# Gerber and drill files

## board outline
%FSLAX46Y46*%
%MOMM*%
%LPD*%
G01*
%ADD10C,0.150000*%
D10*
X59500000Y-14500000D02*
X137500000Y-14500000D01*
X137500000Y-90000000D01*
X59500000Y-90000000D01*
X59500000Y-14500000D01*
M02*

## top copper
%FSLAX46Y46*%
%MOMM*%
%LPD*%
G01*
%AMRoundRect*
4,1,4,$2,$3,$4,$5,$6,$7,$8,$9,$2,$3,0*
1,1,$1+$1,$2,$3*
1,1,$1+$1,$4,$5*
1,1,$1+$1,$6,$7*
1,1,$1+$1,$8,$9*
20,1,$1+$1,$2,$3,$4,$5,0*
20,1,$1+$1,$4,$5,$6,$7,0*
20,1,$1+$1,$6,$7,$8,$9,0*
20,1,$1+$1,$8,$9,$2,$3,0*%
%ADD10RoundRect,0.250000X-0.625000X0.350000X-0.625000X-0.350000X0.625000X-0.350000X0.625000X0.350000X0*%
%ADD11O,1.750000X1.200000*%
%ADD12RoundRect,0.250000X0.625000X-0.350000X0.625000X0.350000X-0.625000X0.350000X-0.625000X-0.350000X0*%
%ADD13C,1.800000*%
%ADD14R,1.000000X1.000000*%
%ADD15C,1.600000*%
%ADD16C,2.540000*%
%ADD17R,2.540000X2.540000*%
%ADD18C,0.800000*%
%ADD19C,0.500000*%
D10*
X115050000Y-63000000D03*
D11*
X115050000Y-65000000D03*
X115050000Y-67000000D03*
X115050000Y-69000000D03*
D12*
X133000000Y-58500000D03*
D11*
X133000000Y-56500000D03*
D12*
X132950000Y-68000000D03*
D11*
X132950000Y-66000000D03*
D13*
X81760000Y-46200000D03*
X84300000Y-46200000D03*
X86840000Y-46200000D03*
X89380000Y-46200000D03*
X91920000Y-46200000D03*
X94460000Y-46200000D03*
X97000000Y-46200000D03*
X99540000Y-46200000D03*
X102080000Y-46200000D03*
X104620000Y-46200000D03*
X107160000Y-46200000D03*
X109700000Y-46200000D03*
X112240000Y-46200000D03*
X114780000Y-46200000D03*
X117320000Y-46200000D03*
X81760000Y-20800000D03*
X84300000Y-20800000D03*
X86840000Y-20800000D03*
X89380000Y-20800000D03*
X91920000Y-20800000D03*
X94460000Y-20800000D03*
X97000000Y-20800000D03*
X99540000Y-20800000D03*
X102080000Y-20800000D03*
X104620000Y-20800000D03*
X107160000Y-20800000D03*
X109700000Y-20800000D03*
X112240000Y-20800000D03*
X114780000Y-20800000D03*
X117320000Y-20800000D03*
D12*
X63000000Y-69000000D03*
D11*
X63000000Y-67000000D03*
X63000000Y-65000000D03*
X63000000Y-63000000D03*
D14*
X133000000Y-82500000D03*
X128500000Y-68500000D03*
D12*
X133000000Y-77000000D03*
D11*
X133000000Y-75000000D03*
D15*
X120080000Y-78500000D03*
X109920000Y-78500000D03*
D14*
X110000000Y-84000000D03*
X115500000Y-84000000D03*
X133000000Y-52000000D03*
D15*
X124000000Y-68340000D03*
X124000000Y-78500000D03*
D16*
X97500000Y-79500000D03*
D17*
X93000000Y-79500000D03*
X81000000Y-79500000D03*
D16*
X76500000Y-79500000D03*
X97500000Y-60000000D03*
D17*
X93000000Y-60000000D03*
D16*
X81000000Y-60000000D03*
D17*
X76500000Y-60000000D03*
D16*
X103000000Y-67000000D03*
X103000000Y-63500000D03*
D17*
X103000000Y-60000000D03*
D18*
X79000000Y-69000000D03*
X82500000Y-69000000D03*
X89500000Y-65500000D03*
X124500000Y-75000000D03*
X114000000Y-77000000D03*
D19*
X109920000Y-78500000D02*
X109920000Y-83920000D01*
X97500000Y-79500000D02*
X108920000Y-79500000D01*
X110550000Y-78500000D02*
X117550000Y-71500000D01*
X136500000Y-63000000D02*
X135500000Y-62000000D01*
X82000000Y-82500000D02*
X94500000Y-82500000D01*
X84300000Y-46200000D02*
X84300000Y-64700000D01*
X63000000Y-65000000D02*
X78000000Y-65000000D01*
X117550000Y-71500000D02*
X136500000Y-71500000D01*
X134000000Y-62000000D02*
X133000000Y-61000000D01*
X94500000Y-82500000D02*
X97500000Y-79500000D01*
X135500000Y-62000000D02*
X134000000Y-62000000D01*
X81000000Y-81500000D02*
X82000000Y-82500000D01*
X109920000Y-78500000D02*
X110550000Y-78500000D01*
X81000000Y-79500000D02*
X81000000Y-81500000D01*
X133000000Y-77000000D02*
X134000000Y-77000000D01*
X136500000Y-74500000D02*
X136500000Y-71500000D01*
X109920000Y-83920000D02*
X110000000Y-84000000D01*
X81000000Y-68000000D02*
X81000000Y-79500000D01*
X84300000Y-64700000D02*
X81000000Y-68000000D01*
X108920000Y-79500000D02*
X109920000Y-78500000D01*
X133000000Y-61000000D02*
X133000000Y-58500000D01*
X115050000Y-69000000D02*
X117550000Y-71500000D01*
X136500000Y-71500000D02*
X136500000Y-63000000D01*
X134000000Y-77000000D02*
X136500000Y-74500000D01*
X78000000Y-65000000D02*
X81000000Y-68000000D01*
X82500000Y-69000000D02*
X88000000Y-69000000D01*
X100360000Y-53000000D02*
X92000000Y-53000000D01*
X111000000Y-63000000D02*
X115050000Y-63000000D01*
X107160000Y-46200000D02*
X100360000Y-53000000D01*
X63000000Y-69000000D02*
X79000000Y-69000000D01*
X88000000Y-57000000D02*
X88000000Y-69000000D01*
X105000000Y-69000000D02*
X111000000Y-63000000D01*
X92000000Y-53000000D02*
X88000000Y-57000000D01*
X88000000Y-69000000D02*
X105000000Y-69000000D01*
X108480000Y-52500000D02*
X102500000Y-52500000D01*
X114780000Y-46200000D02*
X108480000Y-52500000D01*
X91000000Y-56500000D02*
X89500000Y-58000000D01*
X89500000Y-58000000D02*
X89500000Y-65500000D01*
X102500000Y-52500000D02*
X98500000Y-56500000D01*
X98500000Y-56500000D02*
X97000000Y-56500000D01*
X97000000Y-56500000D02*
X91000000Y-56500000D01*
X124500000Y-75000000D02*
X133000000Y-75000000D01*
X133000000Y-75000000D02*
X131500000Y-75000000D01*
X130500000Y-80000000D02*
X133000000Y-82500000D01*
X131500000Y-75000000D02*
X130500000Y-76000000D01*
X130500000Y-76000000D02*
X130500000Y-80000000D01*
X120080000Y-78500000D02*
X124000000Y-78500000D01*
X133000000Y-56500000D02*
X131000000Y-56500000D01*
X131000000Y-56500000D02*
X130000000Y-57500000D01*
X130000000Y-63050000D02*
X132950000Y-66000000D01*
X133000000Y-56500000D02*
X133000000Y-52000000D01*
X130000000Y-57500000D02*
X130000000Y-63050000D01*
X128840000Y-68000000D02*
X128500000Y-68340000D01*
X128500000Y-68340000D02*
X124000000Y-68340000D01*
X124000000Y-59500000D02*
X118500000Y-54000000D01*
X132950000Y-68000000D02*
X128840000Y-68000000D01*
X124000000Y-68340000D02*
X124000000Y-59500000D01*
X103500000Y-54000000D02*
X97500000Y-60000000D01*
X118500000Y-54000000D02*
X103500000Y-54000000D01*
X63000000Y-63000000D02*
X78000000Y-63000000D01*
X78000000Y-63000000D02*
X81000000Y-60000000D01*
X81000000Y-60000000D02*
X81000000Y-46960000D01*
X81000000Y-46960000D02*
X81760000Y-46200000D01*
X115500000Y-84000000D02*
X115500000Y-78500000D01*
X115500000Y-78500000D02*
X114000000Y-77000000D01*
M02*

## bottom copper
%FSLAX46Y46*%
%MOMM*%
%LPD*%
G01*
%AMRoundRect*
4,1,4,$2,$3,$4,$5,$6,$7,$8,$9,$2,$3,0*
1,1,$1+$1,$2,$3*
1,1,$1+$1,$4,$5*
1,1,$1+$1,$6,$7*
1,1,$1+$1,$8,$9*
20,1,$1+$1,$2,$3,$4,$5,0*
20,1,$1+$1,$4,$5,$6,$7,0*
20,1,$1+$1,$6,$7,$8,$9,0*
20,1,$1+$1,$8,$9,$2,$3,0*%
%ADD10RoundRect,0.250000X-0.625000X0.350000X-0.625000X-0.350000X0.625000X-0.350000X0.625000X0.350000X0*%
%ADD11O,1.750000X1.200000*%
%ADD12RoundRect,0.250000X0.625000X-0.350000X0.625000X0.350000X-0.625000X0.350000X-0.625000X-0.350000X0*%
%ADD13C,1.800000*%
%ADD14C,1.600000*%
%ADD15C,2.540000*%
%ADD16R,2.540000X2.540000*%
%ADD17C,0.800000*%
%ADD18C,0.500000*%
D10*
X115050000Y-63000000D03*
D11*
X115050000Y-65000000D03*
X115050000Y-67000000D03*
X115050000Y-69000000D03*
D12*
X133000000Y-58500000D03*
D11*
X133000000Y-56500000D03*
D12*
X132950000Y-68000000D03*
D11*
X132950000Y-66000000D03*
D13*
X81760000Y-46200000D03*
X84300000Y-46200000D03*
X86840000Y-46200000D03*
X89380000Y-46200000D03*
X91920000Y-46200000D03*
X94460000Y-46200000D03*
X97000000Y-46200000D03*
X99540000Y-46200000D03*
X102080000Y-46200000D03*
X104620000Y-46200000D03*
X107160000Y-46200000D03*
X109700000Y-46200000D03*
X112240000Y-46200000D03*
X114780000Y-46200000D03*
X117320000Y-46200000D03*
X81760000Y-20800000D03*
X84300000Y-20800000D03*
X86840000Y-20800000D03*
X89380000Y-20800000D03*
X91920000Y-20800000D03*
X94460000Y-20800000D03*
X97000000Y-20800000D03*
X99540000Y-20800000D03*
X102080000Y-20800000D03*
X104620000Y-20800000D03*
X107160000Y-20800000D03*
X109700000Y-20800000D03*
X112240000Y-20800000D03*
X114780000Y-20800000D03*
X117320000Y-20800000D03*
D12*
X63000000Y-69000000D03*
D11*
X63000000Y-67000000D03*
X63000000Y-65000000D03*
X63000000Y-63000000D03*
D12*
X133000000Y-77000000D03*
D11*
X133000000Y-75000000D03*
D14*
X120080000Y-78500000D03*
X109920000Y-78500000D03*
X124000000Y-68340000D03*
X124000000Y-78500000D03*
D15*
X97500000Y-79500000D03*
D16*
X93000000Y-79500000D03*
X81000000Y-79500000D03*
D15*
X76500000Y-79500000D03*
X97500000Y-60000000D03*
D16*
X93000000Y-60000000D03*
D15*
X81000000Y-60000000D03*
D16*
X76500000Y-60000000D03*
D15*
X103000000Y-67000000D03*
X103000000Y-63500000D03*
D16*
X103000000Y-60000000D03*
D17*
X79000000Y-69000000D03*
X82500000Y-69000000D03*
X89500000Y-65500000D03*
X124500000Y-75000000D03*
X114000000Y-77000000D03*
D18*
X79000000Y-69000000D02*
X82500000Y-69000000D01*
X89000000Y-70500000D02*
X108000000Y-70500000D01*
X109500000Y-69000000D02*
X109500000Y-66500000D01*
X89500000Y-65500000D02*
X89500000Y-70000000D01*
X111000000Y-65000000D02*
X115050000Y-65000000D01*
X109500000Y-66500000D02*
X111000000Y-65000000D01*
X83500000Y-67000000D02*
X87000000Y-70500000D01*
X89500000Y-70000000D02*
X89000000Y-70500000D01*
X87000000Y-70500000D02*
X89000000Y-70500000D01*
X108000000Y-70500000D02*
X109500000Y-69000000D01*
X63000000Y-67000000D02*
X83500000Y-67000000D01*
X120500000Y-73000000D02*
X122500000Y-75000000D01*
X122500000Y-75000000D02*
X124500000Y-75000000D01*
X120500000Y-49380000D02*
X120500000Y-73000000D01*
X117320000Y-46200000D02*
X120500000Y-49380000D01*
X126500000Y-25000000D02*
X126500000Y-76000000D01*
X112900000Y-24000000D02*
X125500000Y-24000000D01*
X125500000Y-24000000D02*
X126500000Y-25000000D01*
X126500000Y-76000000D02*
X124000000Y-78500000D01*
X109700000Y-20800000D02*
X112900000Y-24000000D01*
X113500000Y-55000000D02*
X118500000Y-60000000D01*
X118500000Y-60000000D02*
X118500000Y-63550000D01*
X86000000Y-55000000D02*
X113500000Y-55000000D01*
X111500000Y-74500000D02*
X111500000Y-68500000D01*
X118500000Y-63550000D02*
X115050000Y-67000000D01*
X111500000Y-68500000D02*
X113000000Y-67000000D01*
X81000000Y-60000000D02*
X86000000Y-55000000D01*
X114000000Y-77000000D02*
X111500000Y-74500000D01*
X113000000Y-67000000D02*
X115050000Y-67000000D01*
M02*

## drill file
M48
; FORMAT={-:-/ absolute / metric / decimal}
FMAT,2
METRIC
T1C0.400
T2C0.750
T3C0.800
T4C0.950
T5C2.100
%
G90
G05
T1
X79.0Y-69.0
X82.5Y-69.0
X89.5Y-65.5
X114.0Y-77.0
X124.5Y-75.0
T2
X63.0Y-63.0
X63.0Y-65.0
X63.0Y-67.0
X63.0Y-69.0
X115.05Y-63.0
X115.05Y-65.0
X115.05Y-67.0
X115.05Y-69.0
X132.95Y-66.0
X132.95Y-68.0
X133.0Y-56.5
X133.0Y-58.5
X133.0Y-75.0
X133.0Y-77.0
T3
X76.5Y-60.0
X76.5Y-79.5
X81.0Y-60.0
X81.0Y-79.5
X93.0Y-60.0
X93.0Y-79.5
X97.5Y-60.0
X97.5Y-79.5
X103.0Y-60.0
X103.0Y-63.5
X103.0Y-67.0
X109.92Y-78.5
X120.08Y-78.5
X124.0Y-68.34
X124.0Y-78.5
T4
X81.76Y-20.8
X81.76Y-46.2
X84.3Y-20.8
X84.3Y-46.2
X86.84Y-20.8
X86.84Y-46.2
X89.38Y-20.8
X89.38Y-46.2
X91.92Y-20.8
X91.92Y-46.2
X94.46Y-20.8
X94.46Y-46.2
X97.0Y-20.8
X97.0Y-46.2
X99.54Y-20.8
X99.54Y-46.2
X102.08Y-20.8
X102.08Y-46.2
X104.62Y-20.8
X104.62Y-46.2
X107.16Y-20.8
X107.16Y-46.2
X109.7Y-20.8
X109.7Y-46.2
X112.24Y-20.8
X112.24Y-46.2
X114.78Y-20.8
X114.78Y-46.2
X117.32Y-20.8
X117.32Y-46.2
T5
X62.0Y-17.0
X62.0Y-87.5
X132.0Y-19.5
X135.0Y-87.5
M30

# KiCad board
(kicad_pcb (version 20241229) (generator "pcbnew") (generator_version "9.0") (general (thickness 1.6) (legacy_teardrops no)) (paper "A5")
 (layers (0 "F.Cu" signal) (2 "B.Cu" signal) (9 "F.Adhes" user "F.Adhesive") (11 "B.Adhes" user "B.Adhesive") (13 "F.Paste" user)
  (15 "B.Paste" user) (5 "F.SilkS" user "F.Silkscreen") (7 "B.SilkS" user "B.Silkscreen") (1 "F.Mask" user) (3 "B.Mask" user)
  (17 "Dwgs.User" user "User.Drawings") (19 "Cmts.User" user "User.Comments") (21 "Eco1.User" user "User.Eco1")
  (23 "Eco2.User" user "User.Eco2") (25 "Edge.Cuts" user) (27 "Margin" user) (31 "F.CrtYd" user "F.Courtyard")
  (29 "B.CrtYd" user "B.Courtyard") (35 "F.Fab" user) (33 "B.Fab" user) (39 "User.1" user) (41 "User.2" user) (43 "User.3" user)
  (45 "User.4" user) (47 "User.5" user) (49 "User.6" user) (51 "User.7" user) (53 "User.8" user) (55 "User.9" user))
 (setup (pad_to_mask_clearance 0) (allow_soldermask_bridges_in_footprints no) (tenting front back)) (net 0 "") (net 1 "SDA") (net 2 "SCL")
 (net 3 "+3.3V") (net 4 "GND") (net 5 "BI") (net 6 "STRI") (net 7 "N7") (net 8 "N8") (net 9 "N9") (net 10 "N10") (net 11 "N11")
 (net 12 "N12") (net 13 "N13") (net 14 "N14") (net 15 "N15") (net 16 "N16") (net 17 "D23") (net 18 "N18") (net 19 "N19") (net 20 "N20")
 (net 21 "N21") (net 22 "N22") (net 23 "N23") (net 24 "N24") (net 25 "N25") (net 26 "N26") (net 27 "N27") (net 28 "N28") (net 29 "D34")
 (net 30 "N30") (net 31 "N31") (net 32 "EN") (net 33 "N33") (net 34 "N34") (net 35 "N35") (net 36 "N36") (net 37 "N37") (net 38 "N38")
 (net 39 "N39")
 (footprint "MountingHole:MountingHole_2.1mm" (layer "F.Cu") (at 62 17)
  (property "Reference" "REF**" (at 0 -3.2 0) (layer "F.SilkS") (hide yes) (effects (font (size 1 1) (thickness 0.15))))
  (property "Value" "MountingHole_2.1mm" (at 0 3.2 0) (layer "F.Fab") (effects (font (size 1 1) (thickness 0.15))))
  (pad "" np_thru_hole circle (at 0 0) (size 2.1 2.1) (drill 2.1) (layers "*.Cu" "*.Mask")))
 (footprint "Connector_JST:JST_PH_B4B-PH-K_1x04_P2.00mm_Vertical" (layer "F.Cu") (at 115.05 63 -90)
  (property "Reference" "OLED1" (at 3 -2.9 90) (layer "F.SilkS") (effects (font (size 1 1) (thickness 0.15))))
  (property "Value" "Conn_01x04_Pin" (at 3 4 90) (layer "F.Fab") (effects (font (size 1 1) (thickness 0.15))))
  (pad "1" thru_hole roundrect (at 0 0 270) (size 1.2 1.75) (drill 0.75) (layers "*.Cu" "*.Mask") (remove_unused_layers no)
   (roundrect_rratio 0.208333) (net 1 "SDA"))
  (pad "2" thru_hole oval (at 2 0 270) (size 1.2 1.75) (drill 0.75) (layers "*.Cu" "*.Mask") (remove_unused_layers no) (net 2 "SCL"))
  (pad "3" thru_hole oval (at 4 0 270) (size 1.2 1.75) (drill 0.75) (layers "*.Cu" "*.Mask") (remove_unused_layers no) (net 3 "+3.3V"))
  (pad "4" thru_hole oval (at 6 0 270) (size 1.2 1.75) (drill 0.75) (layers "*.Cu" "*.Mask") (remove_unused_layers no) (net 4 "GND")))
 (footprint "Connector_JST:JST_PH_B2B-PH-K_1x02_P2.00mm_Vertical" (layer "F.Cu") (at 133 58.5 90)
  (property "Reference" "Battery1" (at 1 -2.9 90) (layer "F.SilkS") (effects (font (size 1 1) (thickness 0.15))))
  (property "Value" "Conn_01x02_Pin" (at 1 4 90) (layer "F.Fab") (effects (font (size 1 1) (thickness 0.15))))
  (pad "1" thru_hole roundrect (at 0 0 90) (size 1.2 1.75) (drill 0.75) (layers "*.Cu" "*.Mask") (remove_unused_layers no)
   (roundrect_rratio 0.208333) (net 4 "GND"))
  (pad "2" thru_hole oval (at 2 0 90) (size 1.2 1.75) (drill 0.75) (layers "*.Cu" "*.Mask") (remove_unused_layers no) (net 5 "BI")))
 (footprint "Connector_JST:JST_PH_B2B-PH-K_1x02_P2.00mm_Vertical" (layer "F.Cu") (at 132.95 68 90)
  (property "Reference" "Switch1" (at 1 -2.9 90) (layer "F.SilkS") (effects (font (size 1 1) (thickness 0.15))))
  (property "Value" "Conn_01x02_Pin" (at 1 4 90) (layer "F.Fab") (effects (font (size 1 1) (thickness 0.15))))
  (pad "1" thru_hole roundrect (at 0 0 90) (size 1.2 1.75) (drill 0.75) (layers "*.Cu" "*.Mask") (remove_unused_layers no)
   (roundrect_rratio 0.208333) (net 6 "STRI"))
  (pad "2" thru_hole oval (at 2 0 90) (size 1.2 1.75) (drill 0.75) (layers "*.Cu" "*.Mask") (remove_unused_layers no) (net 5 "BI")))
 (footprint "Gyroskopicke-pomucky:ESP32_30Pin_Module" (layer "F.Cu") (at 104.62 28.42 90)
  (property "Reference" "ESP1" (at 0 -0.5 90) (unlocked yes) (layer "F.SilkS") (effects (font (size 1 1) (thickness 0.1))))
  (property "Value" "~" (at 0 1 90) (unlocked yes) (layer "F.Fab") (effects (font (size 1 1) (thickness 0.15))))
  (pad "1" thru_hole circle (at -17.78 -22.86 90) (size 1.8 1.8) (drill 0.95) (layers "*.Cu" "*.Mask") (remove_unused_layers no)
   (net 3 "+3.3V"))
  (pad "2" thru_hole circle (at -17.78 -20.32 90) (size 1.8 1.8) (drill 0.95) (layers "*.Cu" "*.Mask") (remove_unused_layers no)
   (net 4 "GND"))
  (pad "3" thru_hole circle (at -17.78 -17.78 90) (size 1.8 1.8) (drill 0.95) (layers "*.Cu" "*.Mask") (remove_unused_layers no)
   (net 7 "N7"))
  (pad "4" thru_hole circle (at -17.78 -15.24 90) (size 1.8 1.8) (drill 0.95) (layers "*.Cu" "*.Mask") (remove_unused_layers no)
   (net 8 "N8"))
  (pad "5" thru_hole circle (at -17.78 -12.7 90) (size 1.8 1.8) (drill 0.95) (layers "*.Cu" "*.Mask") (remove_unused_layers no) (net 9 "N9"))
  (pad "6" thru_hole circle (at -17.78 -10.16 90) (size 1.8 1.8) (drill 0.95) (layers "*.Cu" "*.Mask") (remove_unused_layers no)
   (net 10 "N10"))
  (pad "7" thru_hole circle (at -17.78 -7.62 90) (size 1.8 1.8) (drill 0.95) (layers "*.Cu" "*.Mask") (remove_unused_layers no)
   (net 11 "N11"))
  (pad "8" thru_hole circle (at -17.78 -5.08 90) (size 1.8 1.8) (drill 0.95) (layers "*.Cu" "*.Mask") (remove_unused_layers no)
   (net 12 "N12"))
  (pad "9" thru_hole circle (at -17.78 -2.54 90) (size 1.8 1.8) (drill 0.95) (layers "*.Cu" "*.Mask") (remove_unused_layers no)
   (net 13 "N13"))
  (pad "10" thru_hole circle (at -17.78 0 90) (size 1.8 1.8) (drill 0.95) (layers "*.Cu" "*.Mask") (remove_unused_layers no) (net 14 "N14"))
  (pad "11" thru_hole circle (at -17.78 2.54 90) (size 1.8 1.8) (drill 0.95) (layers "*.Cu" "*.Mask") (remove_unused_layers no)
   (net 1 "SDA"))
  (pad "12" thru_hole circle (at -17.78 5.08 90) (size 1.8 1.8) (drill 0.95) (layers "*.Cu" "*.Mask") (remove_unused_layers no)
   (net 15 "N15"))
  (pad "13" thru_hole circle (at -17.78 7.62 90) (size 1.8 1.8) (drill 0.95) (layers "*.Cu" "*.Mask") (remove_unused_layers no)
   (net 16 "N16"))
  (pad "14" thru_hole circle (at -17.78 10.16 90) (size 1.8 1.8) (drill 0.95) (layers "*.Cu" "*.Mask") (remove_unused_layers no)
   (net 2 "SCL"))
  (pad "15" thru_hole circle (at -17.78 12.7 90) (size 1.8 1.8) (drill 0.95) (layers "*.Cu" "*.Mask") (remove_unused_layers no)
   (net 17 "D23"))
  (pad "16" thru_hole circle (at 7.62 -22.86 90) (size 1.8 1.8) (drill 0.95) (layers "*.Cu" "*.Mask") (remove_unused_layers no)
   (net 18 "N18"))
  (pad "17" thru_hole circle (at 7.62 -20.32 90) (size 1.8 1.8) (drill 0.95) (layers "*.Cu" "*.Mask") (remove_unused_layers no)
   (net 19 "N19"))
  (pad "18" thru_hole circle (at 7.62 -17.78 90) (size 1.8 1.8) (drill 0.95) (layers "*.Cu" "*.Mask") (remove_unused_layers no)
   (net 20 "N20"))
  (pad "19" thru_hole circle (at 7.62 -15.24 90) (size 1.8 1.8) (drill 0.95) (layers "*.Cu" "*.Mask") (remove_unused_layers no)
   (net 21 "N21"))
  (pad "20" thru_hole circle (at 7.62 -12.7 90) (size 1.8 1.8) (drill 0.95) (layers "*.Cu" "*.Mask") (remove_unused_layers no)
   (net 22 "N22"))
  (pad "21" thru_hole circle (at 7.62 -10.16 90) (size 1.8 1.8) (drill 0.95) (layers "*.Cu" "*.Mask") (remove_unused_layers no)
   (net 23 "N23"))
  (pad "22" thru_hole circle (at 7.62 -7.62 90) (size 1.8 1.8) (drill 0.95) (layers "*.Cu" "*.Mask") (remove_unused_layers no)
   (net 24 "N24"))
  (pad "23" thru_hole circle (at 7.62 -5.08 90) (size 1.8 1.8) (drill 0.95) (layers "*.Cu" "*.Mask") (remove_unused_layers no)
   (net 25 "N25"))
  (pad "24" thru_hole circle (at 7.62 -2.54 90) (size 1.8 1.8) (drill 0.95) (layers "*.Cu" "*.Mask") (remove_unused_layers no)
   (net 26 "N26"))
  (pad "25" thru_hole circle (at 7.62 0 90) (size 1.8 1.8) (drill 0.95) (layers "*.Cu" "*.Mask") (remove_unused_layers no) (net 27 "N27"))
  (pad "26" thru_hole circle (at 7.62 2.54 90) (size 1.8 1.8) (drill 0.95) (layers "*.Cu" "*.Mask") (remove_unused_layers no) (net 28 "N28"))
  (pad "27" thru_hole circle (at 7.62 5.08 90) (size 1.8 1.8) (drill 0.95) (layers "*.Cu" "*.Mask") (remove_unused_layers no) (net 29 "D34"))
  (pad "28" thru_hole circle (at 7.62 7.62 90) (size 1.8 1.8) (drill 0.95) (layers "*.Cu" "*.Mask") (remove_unused_layers no) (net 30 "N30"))
  (pad "29" thru_hole circle (at 7.62 10.16 90) (size 1.8 1.8) (drill 0.95) (layers "*.Cu" "*.Mask") (remove_unused_layers no)
   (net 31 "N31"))
  (pad "30" thru_hole circle (at 7.62 12.7 90) (size 1.8 1.8) (drill 0.95) (layers "*.Cu" "*.Mask") (remove_unused_layers no) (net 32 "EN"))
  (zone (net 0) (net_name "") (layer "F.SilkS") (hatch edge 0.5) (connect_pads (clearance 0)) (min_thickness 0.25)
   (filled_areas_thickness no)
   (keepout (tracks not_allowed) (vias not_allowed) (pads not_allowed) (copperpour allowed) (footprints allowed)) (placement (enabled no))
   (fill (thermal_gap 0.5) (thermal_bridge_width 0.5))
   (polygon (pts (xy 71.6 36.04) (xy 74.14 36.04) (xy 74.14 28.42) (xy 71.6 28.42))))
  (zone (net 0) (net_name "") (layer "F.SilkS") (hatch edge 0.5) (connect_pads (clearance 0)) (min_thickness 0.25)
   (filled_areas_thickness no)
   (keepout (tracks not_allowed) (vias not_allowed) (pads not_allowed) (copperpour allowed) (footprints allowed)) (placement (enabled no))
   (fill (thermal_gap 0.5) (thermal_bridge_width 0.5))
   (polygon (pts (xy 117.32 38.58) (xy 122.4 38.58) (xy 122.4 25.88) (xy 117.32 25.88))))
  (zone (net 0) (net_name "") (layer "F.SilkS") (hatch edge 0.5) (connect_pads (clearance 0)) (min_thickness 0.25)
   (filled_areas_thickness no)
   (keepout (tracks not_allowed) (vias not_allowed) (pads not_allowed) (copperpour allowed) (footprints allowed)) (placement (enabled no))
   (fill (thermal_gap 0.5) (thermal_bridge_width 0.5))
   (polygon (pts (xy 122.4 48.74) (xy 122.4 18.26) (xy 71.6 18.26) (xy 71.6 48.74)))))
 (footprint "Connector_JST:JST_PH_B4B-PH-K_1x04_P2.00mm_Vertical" (layer "F.Cu") (at 63 69 90)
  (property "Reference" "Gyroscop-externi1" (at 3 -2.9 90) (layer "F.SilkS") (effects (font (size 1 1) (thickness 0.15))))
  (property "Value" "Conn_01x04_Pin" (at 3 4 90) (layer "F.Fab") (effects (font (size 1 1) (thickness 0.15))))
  (pad "1" thru_hole roundrect (at 0 0 90) (size 1.2 1.75) (drill 0.75) (layers "*.Cu" "*.Mask") (remove_unused_layers no)
   (roundrect_rratio 0.208333) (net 1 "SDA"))
  (pad "2" thru_hole oval (at 2 0 90) (size 1.2 1.75) (drill 0.75) (layers "*.Cu" "*.Mask") (remove_unused_layers no) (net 2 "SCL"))
  (pad "3" thru_hole oval (at 4 0 90) (size 1.2 1.75) (drill 0.75) (layers "*.Cu" "*.Mask") (remove_unused_layers no) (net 4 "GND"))
  (pad "4" thru_hole oval (at 6 0 90) (size 1.2 1.75) (drill 0.75) (layers "*.Cu" "*.Mask") (remove_unused_layers no) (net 3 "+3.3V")))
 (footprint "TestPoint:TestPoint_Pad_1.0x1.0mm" (layer "F.Cu") (at 133 82.5)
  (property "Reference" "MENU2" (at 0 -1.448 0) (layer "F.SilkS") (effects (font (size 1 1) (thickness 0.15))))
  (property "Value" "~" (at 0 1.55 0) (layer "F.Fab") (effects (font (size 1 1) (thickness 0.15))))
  (pad "1" smd rect (at 0 0) (size 1 1) (layers "F.Cu" "F.Mask") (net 17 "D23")))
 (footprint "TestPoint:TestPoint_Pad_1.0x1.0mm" (layer "F.Cu") (at 128.5 68.5 90)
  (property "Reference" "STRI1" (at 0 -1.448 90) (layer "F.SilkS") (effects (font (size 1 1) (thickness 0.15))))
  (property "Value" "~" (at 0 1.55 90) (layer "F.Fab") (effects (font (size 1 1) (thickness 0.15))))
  (pad "1" smd rect (at 0 0 90) (size 1 1) (layers "F.Cu" "F.Mask") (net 6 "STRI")))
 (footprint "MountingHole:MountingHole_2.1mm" (layer "F.Cu") (at 62 87.5)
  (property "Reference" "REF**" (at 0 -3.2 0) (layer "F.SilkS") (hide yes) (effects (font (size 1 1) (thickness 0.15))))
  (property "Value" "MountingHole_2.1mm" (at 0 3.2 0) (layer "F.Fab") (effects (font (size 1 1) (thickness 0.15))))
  (pad "" np_thru_hole circle (at 0 0) (size 2.1 2.1) (drill 2.1) (layers "*.Cu" "*.Mask")))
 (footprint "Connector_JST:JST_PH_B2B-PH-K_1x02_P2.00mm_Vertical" (layer "F.Cu") (at 133 77 90)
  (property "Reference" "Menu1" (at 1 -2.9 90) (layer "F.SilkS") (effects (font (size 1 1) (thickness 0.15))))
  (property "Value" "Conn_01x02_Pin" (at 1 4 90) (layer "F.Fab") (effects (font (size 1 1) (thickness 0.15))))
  (pad "1" thru_hole roundrect (at 0 0 90) (size 1.2 1.75) (drill 0.75) (layers "*.Cu" "*.Mask") (remove_unused_layers no)
   (roundrect_rratio 0.208333) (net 4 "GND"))
  (pad "2" thru_hole oval (at 2 0 90) (size 1.2 1.75) (drill 0.75) (layers "*.Cu" "*.Mask") (remove_unused_layers no) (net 17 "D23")))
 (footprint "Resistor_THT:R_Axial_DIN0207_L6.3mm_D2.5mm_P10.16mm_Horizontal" (layer "F.Cu") (at 120.08 78.5 180)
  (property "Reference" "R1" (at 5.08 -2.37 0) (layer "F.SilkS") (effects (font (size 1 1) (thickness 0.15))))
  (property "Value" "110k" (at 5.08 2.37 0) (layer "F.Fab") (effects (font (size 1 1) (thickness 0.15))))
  (pad "1" thru_hole circle (at 0 0 180) (size 1.6 1.6) (drill 0.8) (layers "*.Cu" "*.Mask") (remove_unused_layers no) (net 29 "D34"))
  (pad "2" thru_hole circle (at 10.16 0 180) (size 1.6 1.6) (drill 0.8) (layers "*.Cu" "*.Mask") (remove_unused_layers no) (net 4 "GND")))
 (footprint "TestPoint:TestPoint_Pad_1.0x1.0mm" (layer "F.Cu") (at 110 84)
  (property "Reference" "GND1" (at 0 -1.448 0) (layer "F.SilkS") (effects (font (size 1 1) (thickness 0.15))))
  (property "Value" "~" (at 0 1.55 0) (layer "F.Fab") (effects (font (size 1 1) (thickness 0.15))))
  (pad "1" smd rect (at 0 0) (size 1 1) (layers "F.Cu" "F.Mask") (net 4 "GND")))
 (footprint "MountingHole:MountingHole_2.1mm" (layer "F.Cu") (at 132 19.5)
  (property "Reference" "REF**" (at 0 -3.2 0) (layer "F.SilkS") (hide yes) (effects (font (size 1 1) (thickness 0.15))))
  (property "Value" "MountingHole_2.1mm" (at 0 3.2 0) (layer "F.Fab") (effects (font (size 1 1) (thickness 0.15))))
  (pad "" np_thru_hole circle (at 0 0) (size 2.1 2.1) (drill 2.1) (layers "*.Cu" "*.Mask")))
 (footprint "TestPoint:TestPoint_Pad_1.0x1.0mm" (layer "F.Cu") (at 115.5 84)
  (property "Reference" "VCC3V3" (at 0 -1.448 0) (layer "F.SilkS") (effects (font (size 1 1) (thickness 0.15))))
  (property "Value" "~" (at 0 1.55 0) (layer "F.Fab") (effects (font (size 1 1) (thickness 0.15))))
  (pad "1" smd rect (at 0 0) (size 1 1) (layers "F.Cu" "F.Mask") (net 3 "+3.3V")))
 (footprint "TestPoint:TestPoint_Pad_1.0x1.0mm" (layer "F.Cu") (at 133 52)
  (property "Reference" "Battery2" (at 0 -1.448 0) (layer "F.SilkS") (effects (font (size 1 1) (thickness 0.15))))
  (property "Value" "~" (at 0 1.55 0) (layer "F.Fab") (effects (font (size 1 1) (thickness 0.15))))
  (pad "1" smd rect (at 0 0) (size 1 1) (layers "F.Cu" "F.Mask") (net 5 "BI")))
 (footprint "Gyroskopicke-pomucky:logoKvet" (layer "F.Cu") (at 65.5 51.5)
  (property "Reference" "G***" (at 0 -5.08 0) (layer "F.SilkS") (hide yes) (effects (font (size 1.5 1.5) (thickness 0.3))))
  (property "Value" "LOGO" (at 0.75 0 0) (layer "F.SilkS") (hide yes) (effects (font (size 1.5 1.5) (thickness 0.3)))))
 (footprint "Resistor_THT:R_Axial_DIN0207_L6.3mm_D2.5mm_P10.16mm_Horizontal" (layer "F.Cu") (at 124 68.34 -90)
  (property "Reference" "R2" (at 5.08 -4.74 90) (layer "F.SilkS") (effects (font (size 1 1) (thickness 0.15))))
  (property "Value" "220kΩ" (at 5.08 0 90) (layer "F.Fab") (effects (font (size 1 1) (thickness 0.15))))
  (pad "1" thru_hole circle (at 0 0 270) (size 1.6 1.6) (drill 0.8) (layers "*.Cu" "*.Mask") (remove_unused_layers no) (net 6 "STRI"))
  (pad "2" thru_hole circle (at 10.16 0 270) (size 1.6 1.6) (drill 0.8) (layers "*.Cu" "*.Mask") (remove_unused_layers no) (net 29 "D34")))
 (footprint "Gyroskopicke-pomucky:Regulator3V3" (layer "F.Cu") (at 84.5 70 180)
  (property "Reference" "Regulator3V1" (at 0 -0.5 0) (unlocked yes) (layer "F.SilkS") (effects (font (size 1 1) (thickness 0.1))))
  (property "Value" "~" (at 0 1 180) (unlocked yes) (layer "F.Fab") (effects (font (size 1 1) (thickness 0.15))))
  (pad "1" thru_hole circle (at -13 -9.5 180) (size 2.54 2.54) (drill 0.8) (layers "*.Cu" "*.Mask") (remove_unused_layers no) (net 4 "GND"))
  (pad "2" thru_hole rect (at -8.5 -9.5 180) (size 2.54 2.54) (drill 0.8) (layers "*.Cu" "*.Mask") (remove_unused_layers no) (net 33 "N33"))
  (pad "3" thru_hole rect (at 3.5 -9.5 180) (size 2.54 2.54) (drill 0.8) (layers "*.Cu" "*.Mask") (remove_unused_layers no) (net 4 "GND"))
  (pad "4" thru_hole circle (at 8 -9.5 180) (size 2.54 2.54) (drill 0.8) (layers "*.Cu" "*.Mask") (remove_unused_layers no) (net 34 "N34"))
  (pad "5" thru_hole circle (at -13 10 180) (size 2.54 2.54) (drill 0.8) (layers "*.Cu" "*.Mask") (remove_unused_layers no) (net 6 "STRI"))
  (pad "6" thru_hole rect (at -8.5 10 180) (size 2.54 2.54) (drill 0.8) (layers "*.Cu" "*.Mask") (remove_unused_layers no) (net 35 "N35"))
  (pad "7" thru_hole circle (at 3.5 10 180) (size 2.54 2.54) (drill 0.8) (layers "*.Cu" "*.Mask") (remove_unused_layers no) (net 3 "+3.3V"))
  (pad "8" thru_hole rect (at 8 10 180) (size 2.54 2.54) (drill 0.8) (layers "*.Cu" "*.Mask") (remove_unused_layers no) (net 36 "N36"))
  (pad "9" thru_hole circle (at -18.5 3 180) (size 2.54 2.54) (drill 0.8) (layers "*.Cu" "*.Mask") (remove_unused_layers no) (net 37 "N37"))
  (pad "10" thru_hole circle (at -18.5 6.5 180) (size 2.54 2.54) (drill 0.8) (layers "*.Cu" "*.Mask") (remove_unused_layers no)
   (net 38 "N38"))
  (pad "11" thru_hole rect (at -18.5 10 180) (size 2.54 2.54) (drill 0.8) (layers "*.Cu" "*.Mask") (remove_unused_layers no) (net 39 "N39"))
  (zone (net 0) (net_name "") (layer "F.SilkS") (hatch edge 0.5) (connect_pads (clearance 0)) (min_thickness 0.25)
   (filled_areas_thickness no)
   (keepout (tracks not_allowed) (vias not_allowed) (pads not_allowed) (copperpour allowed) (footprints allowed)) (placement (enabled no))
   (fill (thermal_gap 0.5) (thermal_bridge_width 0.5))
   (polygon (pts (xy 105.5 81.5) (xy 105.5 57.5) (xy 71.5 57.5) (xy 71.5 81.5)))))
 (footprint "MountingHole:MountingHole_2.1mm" (layer "F.Cu") (at 135 87.5)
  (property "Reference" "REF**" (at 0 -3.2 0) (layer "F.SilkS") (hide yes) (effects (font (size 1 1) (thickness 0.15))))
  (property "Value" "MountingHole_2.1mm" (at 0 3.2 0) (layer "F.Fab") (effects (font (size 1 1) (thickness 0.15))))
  (pad "" np_thru_hole circle (at 0 0) (size 2.1 2.1) (drill 2.1) (layers "*.Cu" "*.Mask")))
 (gr_rect (start 59.5 14.5) (end 137.5 90) (stroke (width 0.15) (type solid)) (fill no) (layer "Edge.Cuts"))
 (segment (start 109.92 78.5) (end 109.92 83.92) (width 0.5) (layer "F.Cu") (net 4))
 (segment (start 97.5 79.5) (end 108.92 79.5) (width 0.5) (layer "F.Cu") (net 4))
 (segment (start 110.55 78.5) (end 117.55 71.5) (width 0.5) (layer "F.Cu") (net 4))
 (segment (start 136.5 63) (end 135.5 62) (width 0.5) (layer "F.Cu") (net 4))
 (segment (start 82 82.5) (end 94.5 82.5) (width 0.5) (layer "F.Cu") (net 4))
 (segment (start 84.3 46.2) (end 84.3 64.7) (width 0.5) (layer "F.Cu") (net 4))
 (segment (start 63 65) (end 78 65) (width 0.5) (layer "F.Cu") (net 4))
 (segment (start 117.55 71.5) (end 136.5 71.5) (width 0.5) (layer "F.Cu") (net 4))
 (segment (start 134 62) (end 133 61) (width 0.5) (layer "F.Cu") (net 4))
 (segment (start 94.5 82.5) (end 97.5 79.5) (width 0.5) (layer "F.Cu") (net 4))
 (segment (start 135.5 62) (end 134 62) (width 0.5) (layer "F.Cu") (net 4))
 (segment (start 81 81.5) (end 82 82.5) (width 0.5) (layer "F.Cu") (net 4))
 (segment (start 109.92 78.5) (end 110.55 78.5) (width 0.5) (layer "F.Cu") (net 4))
 (segment (start 81 79.5) (end 81 81.5) (width 0.5) (layer "F.Cu") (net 4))
 (segment (start 133 77) (end 134 77) (width 0.5) (layer "F.Cu") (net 4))
 (segment (start 136.5 74.5) (end 136.5 71.5) (width 0.5) (layer "F.Cu") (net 4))
 (segment (start 109.92 83.92) (end 110 84) (width 0.5) (layer "F.Cu") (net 4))
 (segment (start 81 68) (end 81 79.5) (width 0.5) (layer "F.Cu") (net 4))
 (segment (start 84.3 64.7) (end 81 68) (width 0.5) (layer "F.Cu") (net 4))
 (segment (start 108.92 79.5) (end 109.92 78.5) (width 0.5) (layer "F.Cu") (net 4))
 (segment (start 133 61) (end 133 58.5) (width 0.5) (layer "F.Cu") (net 4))
 (segment (start 115.05 69) (end 117.55 71.5) (width 0.5) (layer "F.Cu") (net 4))
 (segment (start 136.5 71.5) (end 136.5 63) (width 0.5) (layer "F.Cu") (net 4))
 (segment (start 134 77) (end 136.5 74.5) (width 0.5) (layer "F.Cu") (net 4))
 (segment (start 78 65) (end 81 68) (width 0.5) (layer "F.Cu") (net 4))
 (segment (start 82.5 69) (end 88 69) (width 0.5) (layer "F.Cu") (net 1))
 (segment (start 100.36 53) (end 92 53) (width 0.5) (layer "F.Cu") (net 1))
 (segment (start 111 63) (end 115.05 63) (width 0.5) (layer "F.Cu") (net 1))
 (segment (start 107.16 46.2) (end 100.36 53) (width 0.5) (layer "F.Cu") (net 1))
 (segment (start 63 69) (end 79 69) (width 0.5) (layer "F.Cu") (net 1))
 (segment (start 88 57) (end 88 69) (width 0.5) (layer "F.Cu") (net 1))
 (segment (start 105 69) (end 111 63) (width 0.5) (layer "F.Cu") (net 1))
 (segment (start 92 53) (end 88 57) (width 0.5) (layer "F.Cu") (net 1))
 (segment (start 88 69) (end 105 69) (width 0.5) (layer "F.Cu") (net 1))
 (via (at 79 69) (size 0.8) (drill 0.4) (layers "F.Cu" "B.Cu") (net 1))
 (via (at 82.5 69) (size 0.8) (drill 0.4) (layers "F.Cu" "B.Cu") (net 1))
 (segment (start 79 69) (end 82.5 69) (width 0.5) (layer "B.Cu") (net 1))
 (segment (start 108.48 52.5) (end 102.5 52.5) (width 0.5) (layer "F.Cu") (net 2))
 (segment (start 114.78 46.2) (end 108.48 52.5) (width 0.5) (layer "F.Cu") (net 2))
 (segment (start 91 56.5) (end 89.5 58) (width 0.5) (layer "F.Cu") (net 2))
 (segment (start 89.5 58) (end 89.5 65.5) (width 0.5) (layer "F.Cu") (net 2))
 (segment (start 102.5 52.5) (end 98.5 56.5) (width 0.5) (layer "F.Cu") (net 2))
 (segment (start 98.5 56.5) (end 97 56.5) (width 0.5) (layer "F.Cu") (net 2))
 (segment (start 97 56.5) (end 91 56.5) (width 0.5) (layer "F.Cu") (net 2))
 (via (at 89.5 65.5) (size 0.8) (drill 0.4) (layers "F.Cu" "B.Cu") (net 2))
 (segment (start 89 70.5) (end 108 70.5) (width 0.5) (layer "B.Cu") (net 2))
 (segment (start 109.5 69) (end 109.5 66.5) (width 0.5) (layer "B.Cu") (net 2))
 (segment (start 89.5 65.5) (end 89.5 70) (width 0.5) (layer "B.Cu") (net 2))
 (segment (start 111 65) (end 115.05 65) (width 0.5) (layer "B.Cu") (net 2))
 (segment (start 109.5 66.5) (end 111 65) (width 0.5) (layer "B.Cu") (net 2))
 (segment (start 83.5 67) (end 87 70.5) (width 0.5) (layer "B.Cu") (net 2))
 (segment (start 89.5 70) (end 89 70.5) (width 0.5) (layer "B.Cu") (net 2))
 (segment (start 87 70.5) (end 89 70.5) (width 0.5) (layer "B.Cu") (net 2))
 (segment (start 108 70.5) (end 109.5 69) (width 0.5) (layer "B.Cu") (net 2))
 (segment (start 63 67) (end 83.5 67) (width 0.5) (layer "B.Cu") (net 2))
 (segment (start 124.5 75) (end 133 75) (width 0.5) (layer "F.Cu") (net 17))
 (segment (start 133 75) (end 131.5 75) (width 0.5) (layer "F.Cu") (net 17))
 (segment (start 130.5 80) (end 133 82.5) (width 0.5) (layer "F.Cu") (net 17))
 (segment (start 131.5 75) (end 130.5 76) (width 0.5) (layer "F.Cu") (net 17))
 (segment (start 130.5 76) (end 130.5 80) (width 0.5) (layer "F.Cu") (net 17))
 (via (at 124.5 75) (size 0.8) (drill 0.4) (layers "F.Cu" "B.Cu") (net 17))
 (segment (start 120.5 73) (end 122.5 75) (width 0.5) (layer "B.Cu") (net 17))
 (segment (start 122.5 75) (end 124.5 75) (width 0.5) (layer "B.Cu") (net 17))
 (segment (start 120.5 49.38) (end 120.5 73) (width 0.5) (layer "B.Cu") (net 17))
 (segment (start 117.32 46.2) (end 120.5 49.38) (width 0.5) (layer "B.Cu") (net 17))
 (segment (start 120.08 78.5) (end 124 78.5) (width 0.5) (layer "F.Cu") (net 29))
 (segment (start 126.5 25) (end 126.5 76) (width 0.5) (layer "B.Cu") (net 29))
 (segment (start 112.9 24) (end 125.5 24) (width 0.5) (layer "B.Cu") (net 29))
 (segment (start 125.5 24) (end 126.5 25) (width 0.5) (layer "B.Cu") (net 29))
 (segment (start 126.5 76) (end 124 78.5) (width 0.5) (layer "B.Cu") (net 29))
 (segment (start 109.7 20.8) (end 112.9 24) (width 0.5) (layer "B.Cu") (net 29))
 (segment (start 133 56.5) (end 131 56.5) (width 0.5) (layer "F.Cu") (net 5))
 (segment (start 131 56.5) (end 130 57.5) (width 0.5) (layer "F.Cu") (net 5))
 (segment (start 130 63.05) (end 132.95 66) (width 0.5) (layer "F.Cu") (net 5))
 (segment (start 133 56.5) (end 133 52) (width 0.5) (layer "F.Cu") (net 5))
 (segment (start 130 57.5) (end 130 63.05) (width 0.5) (layer "F.Cu") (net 5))
 (segment (start 128.84 68) (end 128.5 68.34) (width 0.5) (layer "F.Cu") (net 6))
 (segment (start 128.5 68.34) (end 124 68.34) (width 0.5) (layer "F.Cu") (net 6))
 (segment (start 124 59.5) (end 118.5 54) (width 0.5) (layer "F.Cu") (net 6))
 (segment (start 132.95 68) (end 128.84 68) (width 0.5) (layer "F.Cu") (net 6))
 (segment (start 124 68.34) (end 124 59.5) (width 0.5) (layer "F.Cu") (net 6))
 (segment (start 103.5 54) (end 97.5 60) (width 0.5) (layer "F.Cu") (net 6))
 (segment (start 118.5 54) (end 103.5 54) (width 0.5) (layer "F.Cu") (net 6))
 (segment (start 63 63) (end 78 63) (width 0.5) (layer "F.Cu") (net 3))
 (segment (start 78 63) (end 81 60) (width 0.5) (layer "F.Cu") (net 3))
 (segment (start 81 60) (end 81 46.96) (width 0.5) (layer "F.Cu") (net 3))
 (segment (start 81 46.96) (end 81.76 46.2) (width 0.5) (layer "F.Cu") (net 3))
 (segment (start 115.5 84) (end 115.5 78.5) (width 0.5) (layer "F.Cu") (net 3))
 (segment (start 115.5 78.5) (end 114 77) (width 0.5) (layer "F.Cu") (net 3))
 (via (at 114 77) (size 0.8) (drill 0.4) (layers "F.Cu" "B.Cu") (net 3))
 (segment (start 113.5 55) (end 118.5 60) (width 0.5) (layer "B.Cu") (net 3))
 (segment (start 118.5 60) (end 118.5 63.55) (width 0.5) (layer "B.Cu") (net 3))
 (segment (start 86 55) (end 113.5 55) (width 0.5) (layer "B.Cu") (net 3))
 (segment (start 111.5 74.5) (end 111.5 68.5) (width 0.5) (layer "B.Cu") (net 3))
 (segment (start 118.5 63.55) (end 115.05 67) (width 0.5) (layer "B.Cu") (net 3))
 (segment (start 111.5 68.5) (end 113 67) (width 0.5) (layer "B.Cu") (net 3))
 (segment (start 81 60) (end 86 55) (width 0.5) (layer "B.Cu") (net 3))
 (segment (start 114 77) (end 111.5 74.5) (width 0.5) (layer "B.Cu") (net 3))
 (segment (start 113 67) (end 115.05 67) (width 0.5) (layer "B.Cu") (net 3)))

